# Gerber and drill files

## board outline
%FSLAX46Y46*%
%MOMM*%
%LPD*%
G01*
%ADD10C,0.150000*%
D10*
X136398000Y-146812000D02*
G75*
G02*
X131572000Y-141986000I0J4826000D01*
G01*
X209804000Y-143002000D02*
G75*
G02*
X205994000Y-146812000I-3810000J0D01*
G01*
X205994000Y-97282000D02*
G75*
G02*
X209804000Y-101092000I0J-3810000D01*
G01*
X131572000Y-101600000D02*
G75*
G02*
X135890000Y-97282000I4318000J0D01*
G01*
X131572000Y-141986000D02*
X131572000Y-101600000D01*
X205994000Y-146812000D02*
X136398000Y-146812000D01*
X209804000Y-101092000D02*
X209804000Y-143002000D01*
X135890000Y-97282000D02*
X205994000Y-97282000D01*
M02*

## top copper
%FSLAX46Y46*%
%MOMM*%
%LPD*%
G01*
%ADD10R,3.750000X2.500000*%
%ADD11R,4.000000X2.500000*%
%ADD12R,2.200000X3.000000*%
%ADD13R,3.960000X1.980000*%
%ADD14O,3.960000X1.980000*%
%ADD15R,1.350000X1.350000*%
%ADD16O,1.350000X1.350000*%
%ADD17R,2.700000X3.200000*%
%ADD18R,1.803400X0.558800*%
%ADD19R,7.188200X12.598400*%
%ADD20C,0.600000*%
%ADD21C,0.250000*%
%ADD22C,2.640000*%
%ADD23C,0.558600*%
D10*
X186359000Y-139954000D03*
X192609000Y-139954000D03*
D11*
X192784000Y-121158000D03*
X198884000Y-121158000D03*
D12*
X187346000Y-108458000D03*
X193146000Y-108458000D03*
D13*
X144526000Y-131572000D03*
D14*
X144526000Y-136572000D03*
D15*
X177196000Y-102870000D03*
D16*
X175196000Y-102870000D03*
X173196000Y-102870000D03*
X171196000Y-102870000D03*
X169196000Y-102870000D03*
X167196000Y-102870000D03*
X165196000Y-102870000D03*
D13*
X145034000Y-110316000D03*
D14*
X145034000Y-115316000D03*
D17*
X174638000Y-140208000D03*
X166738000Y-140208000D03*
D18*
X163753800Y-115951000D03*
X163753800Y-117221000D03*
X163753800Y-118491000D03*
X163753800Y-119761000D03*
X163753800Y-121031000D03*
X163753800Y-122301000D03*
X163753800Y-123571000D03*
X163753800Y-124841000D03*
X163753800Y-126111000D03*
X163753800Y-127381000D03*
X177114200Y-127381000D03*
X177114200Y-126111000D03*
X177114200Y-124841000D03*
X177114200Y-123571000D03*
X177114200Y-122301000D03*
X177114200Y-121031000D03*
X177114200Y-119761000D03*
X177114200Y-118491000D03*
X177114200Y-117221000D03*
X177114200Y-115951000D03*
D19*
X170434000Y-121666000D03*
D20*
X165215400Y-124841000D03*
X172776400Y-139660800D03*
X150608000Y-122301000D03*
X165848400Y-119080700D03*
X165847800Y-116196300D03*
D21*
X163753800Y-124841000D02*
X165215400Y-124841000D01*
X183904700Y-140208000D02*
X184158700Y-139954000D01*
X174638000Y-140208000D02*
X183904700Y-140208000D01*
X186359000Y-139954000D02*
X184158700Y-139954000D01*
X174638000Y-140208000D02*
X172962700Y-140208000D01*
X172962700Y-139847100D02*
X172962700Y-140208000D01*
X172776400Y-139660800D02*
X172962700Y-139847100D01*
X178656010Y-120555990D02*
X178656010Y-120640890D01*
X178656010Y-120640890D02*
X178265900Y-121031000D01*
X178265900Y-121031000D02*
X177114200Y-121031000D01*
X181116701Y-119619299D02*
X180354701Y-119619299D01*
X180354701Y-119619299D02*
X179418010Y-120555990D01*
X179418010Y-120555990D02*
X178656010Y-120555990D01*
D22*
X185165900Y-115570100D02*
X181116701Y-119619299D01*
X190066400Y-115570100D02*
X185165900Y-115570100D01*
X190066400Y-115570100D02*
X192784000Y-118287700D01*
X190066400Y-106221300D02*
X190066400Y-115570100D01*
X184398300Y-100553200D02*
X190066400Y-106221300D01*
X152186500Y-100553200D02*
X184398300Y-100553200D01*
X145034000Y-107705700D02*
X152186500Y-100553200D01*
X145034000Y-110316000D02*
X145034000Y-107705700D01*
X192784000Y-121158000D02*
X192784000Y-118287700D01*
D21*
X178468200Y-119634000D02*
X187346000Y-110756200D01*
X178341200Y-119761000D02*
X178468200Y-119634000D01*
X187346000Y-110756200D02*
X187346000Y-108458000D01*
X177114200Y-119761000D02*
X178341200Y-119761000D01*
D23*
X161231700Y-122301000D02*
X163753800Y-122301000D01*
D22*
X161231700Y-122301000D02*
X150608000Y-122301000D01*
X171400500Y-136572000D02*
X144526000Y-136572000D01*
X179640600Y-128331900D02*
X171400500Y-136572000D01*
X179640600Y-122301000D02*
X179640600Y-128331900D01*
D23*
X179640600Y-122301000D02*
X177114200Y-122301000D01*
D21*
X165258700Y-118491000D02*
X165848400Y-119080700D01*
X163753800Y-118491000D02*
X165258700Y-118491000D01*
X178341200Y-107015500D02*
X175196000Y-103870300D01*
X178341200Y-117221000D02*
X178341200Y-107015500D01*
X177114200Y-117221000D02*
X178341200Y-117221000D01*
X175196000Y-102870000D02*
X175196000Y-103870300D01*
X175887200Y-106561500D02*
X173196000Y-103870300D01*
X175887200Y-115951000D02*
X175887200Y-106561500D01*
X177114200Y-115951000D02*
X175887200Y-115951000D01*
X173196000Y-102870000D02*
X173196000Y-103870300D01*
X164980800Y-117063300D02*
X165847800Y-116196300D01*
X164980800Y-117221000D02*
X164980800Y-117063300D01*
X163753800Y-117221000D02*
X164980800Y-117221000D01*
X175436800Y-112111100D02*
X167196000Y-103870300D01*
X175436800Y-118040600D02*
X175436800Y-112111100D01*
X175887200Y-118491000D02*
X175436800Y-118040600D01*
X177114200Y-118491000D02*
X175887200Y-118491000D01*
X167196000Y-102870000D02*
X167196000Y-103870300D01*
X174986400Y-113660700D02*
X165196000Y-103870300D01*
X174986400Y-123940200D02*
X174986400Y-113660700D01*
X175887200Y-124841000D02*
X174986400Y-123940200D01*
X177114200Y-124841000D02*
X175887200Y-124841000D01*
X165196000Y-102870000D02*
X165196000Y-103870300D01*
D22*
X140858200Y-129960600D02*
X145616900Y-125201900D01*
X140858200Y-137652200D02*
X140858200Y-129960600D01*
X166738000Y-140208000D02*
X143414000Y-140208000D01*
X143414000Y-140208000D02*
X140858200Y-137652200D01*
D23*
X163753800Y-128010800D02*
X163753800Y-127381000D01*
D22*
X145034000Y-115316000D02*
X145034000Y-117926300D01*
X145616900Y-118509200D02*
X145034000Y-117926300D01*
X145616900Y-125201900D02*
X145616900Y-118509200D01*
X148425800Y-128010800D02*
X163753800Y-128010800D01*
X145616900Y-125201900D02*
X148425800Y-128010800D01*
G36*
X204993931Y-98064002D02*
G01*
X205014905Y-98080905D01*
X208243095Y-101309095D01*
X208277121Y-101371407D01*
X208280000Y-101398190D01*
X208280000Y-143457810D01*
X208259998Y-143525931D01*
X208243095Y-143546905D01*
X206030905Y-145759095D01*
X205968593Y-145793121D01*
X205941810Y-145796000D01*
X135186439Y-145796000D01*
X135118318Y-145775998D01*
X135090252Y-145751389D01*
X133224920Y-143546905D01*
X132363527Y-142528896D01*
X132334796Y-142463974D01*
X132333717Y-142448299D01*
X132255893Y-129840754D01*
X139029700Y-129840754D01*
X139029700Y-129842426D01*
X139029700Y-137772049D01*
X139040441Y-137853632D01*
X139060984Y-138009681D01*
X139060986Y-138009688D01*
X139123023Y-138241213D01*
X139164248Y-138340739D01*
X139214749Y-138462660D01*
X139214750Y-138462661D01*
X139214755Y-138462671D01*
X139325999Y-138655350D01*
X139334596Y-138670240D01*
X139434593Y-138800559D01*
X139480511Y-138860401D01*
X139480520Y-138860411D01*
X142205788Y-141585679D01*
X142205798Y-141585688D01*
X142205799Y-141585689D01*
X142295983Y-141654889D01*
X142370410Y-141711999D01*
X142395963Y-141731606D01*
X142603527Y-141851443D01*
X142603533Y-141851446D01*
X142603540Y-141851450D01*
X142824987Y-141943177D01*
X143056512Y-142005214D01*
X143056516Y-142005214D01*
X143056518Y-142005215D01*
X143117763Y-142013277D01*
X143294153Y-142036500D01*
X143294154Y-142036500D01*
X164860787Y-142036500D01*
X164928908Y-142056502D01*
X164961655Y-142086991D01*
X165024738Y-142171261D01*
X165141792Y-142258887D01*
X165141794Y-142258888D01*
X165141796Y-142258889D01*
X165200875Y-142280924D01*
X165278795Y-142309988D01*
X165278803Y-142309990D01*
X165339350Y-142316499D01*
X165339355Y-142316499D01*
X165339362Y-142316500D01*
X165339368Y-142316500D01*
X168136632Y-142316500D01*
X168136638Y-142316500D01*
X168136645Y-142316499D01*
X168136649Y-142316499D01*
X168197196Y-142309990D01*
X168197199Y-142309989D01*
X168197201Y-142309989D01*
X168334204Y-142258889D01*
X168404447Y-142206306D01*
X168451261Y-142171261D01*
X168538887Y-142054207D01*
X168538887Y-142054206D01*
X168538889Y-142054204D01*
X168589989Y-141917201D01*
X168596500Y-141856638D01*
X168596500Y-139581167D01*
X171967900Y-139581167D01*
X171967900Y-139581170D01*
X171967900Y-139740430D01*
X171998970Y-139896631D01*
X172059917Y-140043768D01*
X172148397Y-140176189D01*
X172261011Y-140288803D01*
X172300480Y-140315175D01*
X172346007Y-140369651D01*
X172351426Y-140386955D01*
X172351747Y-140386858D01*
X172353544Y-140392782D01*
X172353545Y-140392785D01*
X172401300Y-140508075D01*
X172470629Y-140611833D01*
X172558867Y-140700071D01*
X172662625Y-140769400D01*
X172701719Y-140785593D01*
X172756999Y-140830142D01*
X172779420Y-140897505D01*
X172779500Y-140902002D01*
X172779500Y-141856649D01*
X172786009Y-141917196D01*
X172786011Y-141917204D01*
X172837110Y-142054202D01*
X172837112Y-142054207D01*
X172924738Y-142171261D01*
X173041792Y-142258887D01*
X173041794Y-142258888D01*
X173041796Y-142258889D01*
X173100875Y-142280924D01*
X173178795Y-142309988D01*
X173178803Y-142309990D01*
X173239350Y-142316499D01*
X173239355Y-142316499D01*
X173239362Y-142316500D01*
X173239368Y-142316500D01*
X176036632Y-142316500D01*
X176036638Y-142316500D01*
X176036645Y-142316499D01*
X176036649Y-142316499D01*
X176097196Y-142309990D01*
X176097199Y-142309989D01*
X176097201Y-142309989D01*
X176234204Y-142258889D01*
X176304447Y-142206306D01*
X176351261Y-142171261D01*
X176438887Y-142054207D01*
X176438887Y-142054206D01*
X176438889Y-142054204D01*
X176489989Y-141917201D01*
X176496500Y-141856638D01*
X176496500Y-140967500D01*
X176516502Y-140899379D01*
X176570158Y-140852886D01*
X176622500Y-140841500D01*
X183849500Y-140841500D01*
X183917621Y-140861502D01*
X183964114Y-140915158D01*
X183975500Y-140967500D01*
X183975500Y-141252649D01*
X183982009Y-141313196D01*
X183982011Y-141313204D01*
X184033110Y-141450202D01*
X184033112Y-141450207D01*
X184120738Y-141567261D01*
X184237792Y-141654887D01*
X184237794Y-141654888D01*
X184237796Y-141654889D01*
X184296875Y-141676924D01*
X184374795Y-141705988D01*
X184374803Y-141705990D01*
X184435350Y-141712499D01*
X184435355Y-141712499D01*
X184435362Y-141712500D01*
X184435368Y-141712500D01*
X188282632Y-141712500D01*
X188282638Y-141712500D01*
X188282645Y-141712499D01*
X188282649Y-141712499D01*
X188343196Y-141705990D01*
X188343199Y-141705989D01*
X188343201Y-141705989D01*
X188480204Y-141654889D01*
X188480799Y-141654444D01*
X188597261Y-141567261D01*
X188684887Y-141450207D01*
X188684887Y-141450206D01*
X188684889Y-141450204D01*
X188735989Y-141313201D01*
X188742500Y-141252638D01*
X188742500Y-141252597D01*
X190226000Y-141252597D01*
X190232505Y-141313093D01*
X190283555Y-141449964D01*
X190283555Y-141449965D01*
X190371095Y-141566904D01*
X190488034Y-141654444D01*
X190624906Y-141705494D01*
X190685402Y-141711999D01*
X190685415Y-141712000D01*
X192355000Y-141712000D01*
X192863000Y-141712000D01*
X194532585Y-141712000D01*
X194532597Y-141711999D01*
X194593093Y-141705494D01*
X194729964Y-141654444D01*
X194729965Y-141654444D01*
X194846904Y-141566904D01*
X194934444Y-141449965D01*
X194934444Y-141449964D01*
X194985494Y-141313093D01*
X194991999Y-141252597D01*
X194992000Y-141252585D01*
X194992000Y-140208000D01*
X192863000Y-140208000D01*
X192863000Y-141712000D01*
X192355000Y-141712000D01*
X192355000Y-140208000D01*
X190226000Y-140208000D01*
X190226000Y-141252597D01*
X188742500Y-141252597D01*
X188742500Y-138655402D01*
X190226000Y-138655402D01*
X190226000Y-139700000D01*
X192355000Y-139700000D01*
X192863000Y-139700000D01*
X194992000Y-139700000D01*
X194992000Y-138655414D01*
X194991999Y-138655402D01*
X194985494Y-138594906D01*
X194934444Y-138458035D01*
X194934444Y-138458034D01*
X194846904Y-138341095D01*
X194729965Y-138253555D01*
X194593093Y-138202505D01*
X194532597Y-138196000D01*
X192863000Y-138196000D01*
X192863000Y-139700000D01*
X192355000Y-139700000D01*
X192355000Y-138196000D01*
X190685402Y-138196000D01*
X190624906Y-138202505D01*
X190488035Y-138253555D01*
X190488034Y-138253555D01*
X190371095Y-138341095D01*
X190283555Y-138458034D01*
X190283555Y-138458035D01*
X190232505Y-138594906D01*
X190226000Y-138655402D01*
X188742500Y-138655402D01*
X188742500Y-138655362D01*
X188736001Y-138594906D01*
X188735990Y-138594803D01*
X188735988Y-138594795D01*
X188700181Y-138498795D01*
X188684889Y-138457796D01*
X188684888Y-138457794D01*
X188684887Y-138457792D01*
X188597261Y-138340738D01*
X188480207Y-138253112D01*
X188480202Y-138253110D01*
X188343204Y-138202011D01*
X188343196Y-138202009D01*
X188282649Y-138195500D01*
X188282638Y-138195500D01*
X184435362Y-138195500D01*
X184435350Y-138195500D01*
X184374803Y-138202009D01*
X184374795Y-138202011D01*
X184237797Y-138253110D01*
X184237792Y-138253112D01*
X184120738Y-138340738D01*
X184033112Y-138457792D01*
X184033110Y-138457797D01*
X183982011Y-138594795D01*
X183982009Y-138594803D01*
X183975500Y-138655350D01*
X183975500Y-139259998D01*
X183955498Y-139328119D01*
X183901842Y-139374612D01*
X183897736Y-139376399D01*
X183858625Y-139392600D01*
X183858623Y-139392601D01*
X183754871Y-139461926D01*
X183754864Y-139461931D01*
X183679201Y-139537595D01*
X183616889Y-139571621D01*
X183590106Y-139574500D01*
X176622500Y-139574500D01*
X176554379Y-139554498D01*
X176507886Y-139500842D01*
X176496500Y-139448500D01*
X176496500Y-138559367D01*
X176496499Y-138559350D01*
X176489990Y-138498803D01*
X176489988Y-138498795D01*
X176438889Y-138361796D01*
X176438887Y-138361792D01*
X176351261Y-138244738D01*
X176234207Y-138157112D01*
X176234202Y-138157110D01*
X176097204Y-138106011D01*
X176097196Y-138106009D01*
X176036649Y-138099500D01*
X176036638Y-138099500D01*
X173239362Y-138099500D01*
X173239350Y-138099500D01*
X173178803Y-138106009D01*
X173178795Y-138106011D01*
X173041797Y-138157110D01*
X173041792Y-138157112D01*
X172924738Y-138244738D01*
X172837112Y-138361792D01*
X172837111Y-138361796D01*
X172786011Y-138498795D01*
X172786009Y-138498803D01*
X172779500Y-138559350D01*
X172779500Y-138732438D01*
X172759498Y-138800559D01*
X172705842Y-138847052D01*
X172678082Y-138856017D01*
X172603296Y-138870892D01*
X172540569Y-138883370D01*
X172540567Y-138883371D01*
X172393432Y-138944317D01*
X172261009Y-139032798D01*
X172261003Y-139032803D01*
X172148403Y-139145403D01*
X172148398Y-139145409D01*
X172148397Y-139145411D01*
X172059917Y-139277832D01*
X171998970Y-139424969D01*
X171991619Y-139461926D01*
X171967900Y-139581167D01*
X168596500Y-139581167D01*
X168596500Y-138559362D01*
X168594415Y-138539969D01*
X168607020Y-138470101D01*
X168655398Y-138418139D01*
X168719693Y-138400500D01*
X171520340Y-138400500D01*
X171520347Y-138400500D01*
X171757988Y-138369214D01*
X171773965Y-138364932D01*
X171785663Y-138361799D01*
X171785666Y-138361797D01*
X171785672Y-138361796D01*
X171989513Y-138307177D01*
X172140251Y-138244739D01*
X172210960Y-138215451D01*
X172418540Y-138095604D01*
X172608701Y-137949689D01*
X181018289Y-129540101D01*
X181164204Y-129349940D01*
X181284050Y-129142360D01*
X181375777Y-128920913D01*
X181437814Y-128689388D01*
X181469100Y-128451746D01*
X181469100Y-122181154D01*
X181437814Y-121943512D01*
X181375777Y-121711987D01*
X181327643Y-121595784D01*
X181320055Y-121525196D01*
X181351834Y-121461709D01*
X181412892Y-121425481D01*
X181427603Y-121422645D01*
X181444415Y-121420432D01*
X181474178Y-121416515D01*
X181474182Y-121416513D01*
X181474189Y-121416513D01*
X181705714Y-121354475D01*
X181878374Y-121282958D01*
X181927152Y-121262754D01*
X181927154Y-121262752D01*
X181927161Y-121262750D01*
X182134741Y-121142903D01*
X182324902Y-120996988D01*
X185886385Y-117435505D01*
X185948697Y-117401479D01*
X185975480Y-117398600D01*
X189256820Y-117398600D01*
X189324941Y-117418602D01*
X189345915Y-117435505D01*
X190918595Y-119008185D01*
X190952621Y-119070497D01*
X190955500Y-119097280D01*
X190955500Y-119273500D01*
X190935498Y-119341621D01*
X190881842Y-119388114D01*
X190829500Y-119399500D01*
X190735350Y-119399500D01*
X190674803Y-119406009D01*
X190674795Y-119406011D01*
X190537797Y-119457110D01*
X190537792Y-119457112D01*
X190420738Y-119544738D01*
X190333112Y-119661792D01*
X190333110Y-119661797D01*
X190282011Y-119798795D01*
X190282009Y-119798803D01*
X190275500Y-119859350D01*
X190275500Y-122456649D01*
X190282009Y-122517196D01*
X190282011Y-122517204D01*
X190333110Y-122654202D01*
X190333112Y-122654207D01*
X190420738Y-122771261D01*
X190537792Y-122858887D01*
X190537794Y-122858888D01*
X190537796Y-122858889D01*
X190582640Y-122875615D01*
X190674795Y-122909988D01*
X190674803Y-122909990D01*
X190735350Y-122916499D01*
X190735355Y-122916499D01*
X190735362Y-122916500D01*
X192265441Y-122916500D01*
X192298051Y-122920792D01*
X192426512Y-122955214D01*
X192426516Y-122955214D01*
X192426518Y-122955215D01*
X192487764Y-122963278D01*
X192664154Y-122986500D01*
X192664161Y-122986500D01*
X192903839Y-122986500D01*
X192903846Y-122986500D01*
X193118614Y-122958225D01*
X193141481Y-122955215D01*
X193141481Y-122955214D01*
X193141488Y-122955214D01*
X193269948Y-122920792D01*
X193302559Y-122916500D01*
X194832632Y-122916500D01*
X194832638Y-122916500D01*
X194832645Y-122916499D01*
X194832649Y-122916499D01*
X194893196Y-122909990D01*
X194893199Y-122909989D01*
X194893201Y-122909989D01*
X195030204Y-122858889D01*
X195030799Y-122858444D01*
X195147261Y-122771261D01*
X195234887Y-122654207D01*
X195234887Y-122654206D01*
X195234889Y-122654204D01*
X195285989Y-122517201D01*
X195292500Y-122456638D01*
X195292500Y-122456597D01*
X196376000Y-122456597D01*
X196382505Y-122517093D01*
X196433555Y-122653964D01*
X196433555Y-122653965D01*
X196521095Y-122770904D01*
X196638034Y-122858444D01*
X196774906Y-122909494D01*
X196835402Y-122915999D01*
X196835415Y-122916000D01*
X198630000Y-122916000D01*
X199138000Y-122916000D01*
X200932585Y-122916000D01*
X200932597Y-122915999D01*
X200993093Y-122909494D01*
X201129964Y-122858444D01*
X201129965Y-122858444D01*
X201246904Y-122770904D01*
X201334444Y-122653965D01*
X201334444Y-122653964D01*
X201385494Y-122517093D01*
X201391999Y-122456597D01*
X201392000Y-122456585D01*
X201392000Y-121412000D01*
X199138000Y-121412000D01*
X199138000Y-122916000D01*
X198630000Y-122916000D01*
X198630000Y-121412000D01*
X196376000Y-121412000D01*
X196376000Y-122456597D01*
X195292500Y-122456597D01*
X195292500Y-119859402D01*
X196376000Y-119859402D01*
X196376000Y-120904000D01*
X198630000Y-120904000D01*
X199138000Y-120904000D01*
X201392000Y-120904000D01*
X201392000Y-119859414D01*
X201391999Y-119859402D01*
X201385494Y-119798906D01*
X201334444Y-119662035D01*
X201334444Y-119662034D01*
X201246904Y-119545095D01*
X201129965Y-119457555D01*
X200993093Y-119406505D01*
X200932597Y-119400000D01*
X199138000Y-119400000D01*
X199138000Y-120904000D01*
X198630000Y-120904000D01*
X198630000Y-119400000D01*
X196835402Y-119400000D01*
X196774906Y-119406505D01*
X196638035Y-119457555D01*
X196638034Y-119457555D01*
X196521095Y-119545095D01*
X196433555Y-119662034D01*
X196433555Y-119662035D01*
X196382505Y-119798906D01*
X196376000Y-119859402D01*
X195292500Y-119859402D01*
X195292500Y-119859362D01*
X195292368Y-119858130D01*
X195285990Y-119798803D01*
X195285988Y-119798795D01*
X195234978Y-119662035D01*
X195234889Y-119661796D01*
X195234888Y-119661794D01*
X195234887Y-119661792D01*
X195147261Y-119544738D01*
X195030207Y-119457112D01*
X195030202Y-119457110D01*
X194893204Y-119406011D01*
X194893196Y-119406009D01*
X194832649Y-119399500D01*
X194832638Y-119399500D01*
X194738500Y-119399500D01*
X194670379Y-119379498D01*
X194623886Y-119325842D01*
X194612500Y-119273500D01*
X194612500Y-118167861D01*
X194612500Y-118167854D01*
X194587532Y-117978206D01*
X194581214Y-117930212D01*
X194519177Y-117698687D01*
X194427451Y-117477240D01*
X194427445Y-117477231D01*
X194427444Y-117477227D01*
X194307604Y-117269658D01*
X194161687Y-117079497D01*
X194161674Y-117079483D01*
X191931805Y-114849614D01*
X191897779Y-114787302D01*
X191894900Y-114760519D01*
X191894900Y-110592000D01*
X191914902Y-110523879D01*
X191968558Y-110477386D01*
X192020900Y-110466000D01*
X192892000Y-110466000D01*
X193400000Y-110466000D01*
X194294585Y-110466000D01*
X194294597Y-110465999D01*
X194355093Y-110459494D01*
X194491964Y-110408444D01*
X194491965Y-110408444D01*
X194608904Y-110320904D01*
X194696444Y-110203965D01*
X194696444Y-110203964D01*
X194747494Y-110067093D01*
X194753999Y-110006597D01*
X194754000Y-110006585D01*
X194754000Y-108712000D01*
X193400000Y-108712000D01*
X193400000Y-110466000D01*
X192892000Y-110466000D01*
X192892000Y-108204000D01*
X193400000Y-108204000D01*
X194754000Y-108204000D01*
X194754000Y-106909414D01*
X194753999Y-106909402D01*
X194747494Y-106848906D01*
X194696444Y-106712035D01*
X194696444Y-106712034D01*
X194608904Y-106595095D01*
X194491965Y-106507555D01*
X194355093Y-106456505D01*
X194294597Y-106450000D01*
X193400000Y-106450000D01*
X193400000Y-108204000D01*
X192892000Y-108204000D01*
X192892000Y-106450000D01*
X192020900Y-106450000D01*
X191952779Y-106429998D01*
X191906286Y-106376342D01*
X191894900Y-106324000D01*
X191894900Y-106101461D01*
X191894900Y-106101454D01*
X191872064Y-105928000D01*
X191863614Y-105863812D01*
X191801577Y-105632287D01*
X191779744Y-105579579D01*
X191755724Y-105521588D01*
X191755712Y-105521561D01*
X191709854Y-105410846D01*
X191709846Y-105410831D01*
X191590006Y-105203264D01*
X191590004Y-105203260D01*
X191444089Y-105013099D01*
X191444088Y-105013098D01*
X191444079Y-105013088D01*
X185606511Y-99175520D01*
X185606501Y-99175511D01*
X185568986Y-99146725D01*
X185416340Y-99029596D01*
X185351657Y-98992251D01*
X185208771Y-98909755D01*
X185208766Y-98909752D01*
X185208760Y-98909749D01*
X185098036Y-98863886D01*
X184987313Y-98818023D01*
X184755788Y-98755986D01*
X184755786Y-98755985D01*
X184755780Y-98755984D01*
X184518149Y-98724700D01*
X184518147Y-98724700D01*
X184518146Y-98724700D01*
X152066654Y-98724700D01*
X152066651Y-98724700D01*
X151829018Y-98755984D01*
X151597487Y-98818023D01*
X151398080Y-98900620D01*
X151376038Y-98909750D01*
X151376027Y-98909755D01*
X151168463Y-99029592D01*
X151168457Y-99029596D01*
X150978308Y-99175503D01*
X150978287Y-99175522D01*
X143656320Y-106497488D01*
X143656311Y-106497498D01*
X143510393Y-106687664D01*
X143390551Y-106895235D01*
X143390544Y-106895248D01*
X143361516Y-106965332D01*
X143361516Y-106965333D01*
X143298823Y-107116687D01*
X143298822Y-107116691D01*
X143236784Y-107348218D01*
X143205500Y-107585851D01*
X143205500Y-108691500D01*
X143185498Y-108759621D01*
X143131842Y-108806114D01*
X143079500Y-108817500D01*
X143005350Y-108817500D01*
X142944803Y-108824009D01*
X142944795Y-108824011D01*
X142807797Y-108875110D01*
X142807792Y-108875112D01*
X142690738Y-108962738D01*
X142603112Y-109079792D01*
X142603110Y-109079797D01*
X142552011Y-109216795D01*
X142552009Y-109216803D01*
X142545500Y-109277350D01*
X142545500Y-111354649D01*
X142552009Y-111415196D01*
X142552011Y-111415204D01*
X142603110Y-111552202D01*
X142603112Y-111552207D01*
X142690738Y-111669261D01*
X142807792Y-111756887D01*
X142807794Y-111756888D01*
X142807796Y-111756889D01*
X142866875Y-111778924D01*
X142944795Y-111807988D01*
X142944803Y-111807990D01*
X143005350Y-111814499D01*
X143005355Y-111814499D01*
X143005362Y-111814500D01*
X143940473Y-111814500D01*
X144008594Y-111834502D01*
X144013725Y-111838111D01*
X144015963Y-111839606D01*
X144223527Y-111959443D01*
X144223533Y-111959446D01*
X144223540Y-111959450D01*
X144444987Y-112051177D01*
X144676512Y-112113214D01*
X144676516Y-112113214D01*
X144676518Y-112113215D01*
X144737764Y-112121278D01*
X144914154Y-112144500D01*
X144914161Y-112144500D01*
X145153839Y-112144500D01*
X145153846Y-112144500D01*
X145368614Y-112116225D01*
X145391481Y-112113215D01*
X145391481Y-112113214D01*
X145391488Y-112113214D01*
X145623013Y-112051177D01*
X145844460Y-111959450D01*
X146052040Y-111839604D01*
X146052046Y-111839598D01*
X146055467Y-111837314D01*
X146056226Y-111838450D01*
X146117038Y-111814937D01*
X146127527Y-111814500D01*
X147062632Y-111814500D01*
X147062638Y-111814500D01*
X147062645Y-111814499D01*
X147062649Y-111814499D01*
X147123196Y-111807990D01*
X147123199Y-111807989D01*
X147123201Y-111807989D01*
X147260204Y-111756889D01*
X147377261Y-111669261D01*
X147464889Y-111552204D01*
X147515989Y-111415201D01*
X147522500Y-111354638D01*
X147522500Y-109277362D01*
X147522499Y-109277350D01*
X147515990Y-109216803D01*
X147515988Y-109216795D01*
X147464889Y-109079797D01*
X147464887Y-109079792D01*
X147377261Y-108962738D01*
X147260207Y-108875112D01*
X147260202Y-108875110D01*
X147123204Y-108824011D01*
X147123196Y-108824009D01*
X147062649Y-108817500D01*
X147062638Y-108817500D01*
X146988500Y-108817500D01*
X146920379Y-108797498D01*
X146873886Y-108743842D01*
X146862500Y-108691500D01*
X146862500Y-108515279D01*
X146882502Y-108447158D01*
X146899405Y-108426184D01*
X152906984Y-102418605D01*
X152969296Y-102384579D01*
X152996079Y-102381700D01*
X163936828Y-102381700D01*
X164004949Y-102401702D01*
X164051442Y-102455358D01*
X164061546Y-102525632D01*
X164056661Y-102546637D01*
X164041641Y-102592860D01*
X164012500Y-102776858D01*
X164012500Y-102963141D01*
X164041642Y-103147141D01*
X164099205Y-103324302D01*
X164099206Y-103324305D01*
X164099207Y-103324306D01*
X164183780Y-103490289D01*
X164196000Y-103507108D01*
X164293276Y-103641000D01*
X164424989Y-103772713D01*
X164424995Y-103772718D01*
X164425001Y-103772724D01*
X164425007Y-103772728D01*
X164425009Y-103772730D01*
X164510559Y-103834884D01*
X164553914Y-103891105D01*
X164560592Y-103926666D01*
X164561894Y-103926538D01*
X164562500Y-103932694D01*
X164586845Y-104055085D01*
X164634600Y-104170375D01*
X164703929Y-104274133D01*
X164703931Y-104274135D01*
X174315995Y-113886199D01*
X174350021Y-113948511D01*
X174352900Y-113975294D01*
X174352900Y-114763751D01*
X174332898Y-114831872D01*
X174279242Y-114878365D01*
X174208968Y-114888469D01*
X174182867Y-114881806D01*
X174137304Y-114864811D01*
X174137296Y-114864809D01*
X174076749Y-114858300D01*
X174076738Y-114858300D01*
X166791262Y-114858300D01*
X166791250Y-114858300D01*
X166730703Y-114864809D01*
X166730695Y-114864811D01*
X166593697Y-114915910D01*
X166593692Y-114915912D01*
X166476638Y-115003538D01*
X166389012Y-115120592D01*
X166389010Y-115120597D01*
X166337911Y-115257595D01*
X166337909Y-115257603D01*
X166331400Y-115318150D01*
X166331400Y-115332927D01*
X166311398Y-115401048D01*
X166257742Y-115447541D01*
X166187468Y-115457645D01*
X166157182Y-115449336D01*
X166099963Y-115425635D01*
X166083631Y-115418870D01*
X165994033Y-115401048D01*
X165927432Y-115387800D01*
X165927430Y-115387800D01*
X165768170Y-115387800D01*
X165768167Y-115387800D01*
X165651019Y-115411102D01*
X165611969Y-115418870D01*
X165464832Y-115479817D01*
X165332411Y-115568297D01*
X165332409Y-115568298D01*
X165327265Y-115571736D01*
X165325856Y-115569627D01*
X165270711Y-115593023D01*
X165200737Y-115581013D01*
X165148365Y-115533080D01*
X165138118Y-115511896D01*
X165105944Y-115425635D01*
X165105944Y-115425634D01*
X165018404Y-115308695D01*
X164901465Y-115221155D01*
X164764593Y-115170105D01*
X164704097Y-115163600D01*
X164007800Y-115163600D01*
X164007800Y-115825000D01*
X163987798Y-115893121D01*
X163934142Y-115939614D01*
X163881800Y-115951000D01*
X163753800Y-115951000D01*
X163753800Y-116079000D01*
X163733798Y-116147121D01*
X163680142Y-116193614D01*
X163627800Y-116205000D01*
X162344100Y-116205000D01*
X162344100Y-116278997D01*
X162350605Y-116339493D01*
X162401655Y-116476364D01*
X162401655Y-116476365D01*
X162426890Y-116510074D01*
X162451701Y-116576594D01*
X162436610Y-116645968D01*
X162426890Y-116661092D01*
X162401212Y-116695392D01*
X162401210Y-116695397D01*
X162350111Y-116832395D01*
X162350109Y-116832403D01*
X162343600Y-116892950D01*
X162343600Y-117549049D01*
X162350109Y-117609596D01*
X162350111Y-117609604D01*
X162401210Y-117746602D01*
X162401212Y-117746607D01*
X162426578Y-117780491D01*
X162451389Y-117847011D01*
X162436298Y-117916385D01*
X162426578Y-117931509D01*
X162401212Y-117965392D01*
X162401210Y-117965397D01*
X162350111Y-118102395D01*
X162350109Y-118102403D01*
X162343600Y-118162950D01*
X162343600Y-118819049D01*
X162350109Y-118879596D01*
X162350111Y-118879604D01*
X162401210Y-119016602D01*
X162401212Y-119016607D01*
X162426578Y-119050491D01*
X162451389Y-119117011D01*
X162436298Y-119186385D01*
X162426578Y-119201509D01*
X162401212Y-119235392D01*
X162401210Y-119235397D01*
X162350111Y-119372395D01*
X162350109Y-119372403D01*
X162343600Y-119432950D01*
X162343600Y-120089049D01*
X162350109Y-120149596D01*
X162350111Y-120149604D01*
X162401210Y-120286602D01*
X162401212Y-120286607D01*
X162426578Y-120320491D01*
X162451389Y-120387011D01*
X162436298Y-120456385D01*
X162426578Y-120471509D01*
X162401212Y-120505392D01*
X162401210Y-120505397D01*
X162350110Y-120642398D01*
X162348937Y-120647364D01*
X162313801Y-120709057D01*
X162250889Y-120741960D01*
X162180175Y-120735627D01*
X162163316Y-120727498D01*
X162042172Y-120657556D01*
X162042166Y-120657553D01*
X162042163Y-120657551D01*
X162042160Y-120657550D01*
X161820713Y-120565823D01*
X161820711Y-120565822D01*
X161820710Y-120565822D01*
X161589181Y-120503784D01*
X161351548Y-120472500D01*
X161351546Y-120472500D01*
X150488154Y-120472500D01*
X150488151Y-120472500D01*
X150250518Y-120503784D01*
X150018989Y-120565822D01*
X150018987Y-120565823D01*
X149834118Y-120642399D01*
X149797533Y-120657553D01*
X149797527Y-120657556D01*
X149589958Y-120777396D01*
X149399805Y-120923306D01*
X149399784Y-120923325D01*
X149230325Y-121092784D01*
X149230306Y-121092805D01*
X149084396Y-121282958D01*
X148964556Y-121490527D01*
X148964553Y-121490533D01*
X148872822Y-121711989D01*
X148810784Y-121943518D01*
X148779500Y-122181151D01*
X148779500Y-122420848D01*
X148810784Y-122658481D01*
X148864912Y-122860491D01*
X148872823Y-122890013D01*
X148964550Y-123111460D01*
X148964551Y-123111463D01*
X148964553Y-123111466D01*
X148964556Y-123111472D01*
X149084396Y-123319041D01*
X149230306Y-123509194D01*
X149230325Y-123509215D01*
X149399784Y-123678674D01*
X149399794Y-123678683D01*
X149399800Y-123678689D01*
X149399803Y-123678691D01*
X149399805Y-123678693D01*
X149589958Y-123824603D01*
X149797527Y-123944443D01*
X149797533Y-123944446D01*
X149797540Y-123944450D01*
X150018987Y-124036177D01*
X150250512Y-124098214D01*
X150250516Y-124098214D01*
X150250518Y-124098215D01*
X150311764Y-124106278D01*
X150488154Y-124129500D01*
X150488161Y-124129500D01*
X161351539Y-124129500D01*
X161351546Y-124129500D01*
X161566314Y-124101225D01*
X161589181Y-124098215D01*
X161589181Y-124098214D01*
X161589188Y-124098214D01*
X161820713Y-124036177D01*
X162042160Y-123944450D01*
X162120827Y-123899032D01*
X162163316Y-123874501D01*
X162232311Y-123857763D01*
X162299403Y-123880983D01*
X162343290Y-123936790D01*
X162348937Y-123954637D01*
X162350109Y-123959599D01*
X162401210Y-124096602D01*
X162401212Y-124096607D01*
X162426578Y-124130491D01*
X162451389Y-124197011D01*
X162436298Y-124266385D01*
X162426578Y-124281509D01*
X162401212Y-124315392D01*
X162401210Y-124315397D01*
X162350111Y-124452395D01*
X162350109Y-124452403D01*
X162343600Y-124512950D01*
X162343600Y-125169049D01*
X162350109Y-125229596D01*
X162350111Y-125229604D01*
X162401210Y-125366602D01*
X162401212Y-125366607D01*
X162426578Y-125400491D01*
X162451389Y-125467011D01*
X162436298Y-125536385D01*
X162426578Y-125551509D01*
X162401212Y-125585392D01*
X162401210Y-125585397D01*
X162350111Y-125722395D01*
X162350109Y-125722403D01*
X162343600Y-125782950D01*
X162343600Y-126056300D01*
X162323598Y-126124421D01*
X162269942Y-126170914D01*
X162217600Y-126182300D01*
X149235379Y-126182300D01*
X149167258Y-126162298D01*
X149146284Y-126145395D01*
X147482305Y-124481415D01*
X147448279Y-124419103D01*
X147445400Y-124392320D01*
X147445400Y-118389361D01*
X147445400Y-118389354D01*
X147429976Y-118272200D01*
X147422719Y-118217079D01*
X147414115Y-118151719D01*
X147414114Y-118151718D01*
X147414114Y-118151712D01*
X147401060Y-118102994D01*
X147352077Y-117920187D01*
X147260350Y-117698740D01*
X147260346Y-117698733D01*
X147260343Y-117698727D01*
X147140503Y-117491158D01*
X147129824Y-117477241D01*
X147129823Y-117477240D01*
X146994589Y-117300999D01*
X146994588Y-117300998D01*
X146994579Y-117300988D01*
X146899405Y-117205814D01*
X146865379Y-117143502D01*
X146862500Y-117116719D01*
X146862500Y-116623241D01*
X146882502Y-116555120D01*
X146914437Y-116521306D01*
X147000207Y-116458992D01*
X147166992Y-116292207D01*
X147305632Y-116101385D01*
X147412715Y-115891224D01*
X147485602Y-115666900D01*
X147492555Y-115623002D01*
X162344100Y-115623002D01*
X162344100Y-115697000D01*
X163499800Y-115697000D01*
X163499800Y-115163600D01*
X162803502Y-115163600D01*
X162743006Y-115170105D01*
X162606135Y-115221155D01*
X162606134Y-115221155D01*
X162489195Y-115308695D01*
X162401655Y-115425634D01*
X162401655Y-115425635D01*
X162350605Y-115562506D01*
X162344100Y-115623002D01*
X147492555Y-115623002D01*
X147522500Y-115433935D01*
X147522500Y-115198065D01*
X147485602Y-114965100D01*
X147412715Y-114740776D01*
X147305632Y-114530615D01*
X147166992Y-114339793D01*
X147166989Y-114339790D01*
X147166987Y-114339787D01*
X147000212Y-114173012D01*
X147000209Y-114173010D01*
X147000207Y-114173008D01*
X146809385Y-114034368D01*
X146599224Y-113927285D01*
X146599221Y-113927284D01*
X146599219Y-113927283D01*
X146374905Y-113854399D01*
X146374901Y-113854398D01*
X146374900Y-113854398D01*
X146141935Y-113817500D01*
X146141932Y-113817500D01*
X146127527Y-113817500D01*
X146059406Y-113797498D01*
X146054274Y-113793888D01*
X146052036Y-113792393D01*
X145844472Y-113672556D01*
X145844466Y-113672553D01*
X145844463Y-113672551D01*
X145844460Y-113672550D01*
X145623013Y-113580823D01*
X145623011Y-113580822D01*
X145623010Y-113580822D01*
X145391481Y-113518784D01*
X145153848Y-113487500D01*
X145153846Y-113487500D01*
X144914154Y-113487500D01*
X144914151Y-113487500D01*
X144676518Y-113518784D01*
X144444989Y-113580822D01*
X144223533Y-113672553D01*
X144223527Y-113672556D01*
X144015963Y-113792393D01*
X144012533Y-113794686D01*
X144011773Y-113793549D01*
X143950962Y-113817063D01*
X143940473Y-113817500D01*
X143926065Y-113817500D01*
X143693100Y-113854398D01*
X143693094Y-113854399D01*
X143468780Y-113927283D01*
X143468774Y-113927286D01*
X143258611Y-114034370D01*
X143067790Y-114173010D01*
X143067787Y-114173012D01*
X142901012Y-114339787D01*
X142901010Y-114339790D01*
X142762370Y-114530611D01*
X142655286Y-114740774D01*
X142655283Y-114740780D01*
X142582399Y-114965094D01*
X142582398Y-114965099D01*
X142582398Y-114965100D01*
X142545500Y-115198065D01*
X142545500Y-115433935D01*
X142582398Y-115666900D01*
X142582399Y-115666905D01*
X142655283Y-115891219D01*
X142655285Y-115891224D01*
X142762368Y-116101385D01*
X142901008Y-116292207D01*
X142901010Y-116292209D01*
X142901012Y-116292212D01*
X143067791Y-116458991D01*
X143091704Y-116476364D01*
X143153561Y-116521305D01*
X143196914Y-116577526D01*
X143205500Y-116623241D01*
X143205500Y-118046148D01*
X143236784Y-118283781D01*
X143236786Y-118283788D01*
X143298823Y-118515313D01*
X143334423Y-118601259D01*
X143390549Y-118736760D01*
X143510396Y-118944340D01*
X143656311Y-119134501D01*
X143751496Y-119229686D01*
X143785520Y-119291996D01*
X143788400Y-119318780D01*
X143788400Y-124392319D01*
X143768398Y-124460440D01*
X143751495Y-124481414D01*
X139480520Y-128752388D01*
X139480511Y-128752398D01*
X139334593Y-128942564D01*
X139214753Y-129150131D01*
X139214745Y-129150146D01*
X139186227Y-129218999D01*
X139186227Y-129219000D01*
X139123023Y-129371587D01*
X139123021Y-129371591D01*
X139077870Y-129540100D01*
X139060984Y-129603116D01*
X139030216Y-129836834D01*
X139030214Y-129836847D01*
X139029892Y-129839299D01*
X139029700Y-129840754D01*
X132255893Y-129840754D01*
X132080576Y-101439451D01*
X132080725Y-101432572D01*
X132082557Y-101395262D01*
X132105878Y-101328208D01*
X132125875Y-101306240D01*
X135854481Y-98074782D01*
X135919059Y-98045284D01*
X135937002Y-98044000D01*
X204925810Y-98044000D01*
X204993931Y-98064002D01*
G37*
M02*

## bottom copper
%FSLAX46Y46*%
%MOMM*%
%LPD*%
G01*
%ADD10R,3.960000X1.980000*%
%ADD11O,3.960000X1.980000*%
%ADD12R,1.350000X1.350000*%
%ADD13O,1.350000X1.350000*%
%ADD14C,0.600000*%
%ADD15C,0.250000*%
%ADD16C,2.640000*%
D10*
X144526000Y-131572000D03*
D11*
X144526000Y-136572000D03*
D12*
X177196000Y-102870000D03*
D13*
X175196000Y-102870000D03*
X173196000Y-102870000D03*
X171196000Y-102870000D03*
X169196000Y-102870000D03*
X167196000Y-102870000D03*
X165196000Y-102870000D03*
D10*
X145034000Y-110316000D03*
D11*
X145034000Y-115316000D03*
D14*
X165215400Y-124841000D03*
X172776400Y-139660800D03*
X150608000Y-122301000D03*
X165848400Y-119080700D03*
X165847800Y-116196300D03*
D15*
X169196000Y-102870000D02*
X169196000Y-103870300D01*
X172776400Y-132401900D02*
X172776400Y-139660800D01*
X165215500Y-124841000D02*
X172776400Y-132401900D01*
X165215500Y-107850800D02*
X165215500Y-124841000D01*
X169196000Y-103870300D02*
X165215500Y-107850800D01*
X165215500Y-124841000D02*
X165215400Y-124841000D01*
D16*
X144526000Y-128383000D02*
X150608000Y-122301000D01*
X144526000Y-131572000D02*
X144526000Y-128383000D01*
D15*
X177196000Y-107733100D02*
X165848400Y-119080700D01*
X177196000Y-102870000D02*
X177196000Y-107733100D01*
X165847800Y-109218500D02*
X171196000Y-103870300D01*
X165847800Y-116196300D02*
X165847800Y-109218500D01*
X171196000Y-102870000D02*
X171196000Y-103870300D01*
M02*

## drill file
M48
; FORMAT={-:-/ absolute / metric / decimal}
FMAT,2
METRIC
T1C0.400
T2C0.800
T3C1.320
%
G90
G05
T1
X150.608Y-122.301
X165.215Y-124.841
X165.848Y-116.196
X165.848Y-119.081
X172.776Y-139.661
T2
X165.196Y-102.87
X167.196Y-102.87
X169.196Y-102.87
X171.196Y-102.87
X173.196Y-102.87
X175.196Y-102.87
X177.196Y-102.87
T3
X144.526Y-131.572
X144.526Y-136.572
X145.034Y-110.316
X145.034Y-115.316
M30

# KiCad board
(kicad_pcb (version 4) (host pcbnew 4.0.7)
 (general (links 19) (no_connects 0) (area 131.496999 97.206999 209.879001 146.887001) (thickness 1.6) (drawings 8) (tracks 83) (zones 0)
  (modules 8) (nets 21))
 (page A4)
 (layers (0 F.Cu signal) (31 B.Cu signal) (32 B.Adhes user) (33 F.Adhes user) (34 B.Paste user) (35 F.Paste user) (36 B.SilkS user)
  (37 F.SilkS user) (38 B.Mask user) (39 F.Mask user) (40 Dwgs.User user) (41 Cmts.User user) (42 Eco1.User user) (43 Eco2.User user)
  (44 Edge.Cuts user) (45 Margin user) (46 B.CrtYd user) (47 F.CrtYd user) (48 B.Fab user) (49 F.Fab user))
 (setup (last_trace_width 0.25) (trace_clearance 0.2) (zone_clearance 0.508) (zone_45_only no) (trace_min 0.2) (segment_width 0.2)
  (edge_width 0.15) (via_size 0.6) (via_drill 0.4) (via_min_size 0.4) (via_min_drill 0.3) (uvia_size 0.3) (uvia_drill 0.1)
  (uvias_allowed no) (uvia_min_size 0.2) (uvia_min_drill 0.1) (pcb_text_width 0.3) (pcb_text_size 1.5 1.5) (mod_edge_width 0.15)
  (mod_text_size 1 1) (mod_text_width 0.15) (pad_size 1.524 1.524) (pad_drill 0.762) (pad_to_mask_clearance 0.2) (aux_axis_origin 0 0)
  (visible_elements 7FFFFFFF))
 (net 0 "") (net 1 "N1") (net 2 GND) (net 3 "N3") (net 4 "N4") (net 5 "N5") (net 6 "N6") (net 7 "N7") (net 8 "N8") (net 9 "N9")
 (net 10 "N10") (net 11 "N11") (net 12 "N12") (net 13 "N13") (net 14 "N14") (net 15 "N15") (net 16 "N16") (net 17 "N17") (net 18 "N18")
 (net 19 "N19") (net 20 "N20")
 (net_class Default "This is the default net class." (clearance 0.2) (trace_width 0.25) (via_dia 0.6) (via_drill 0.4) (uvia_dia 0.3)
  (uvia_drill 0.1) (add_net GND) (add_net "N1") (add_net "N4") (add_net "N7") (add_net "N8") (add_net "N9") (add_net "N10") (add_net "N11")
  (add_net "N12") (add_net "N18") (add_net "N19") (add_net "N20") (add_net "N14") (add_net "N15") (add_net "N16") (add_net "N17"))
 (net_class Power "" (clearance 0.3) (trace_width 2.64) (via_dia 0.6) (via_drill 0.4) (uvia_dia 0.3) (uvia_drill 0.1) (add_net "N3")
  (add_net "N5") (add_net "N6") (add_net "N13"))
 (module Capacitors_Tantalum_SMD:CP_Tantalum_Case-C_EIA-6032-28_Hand (layer F.Cu) (at 189.484 139.954)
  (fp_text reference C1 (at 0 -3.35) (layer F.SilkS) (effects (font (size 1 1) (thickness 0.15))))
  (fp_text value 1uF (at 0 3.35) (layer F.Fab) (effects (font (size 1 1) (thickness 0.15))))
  (pad 1 smd rect (at -3.125 0) (size 3.75 2.5) (layers F.Cu F.Paste F.Mask) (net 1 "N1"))
  (pad 2 smd rect (at 3.125 0) (size 3.75 2.5) (layers F.Cu F.Paste F.Mask) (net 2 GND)))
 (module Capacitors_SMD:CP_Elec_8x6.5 (layer F.Cu) (at 195.834 121.158)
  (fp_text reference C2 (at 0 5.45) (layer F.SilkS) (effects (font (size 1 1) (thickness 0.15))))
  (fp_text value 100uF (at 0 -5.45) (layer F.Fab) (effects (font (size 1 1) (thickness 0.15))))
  (pad 1 smd rect (at -3.05 0 180) (size 4 2.5) (layers F.Cu F.Paste F.Mask) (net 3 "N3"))
  (pad 2 smd rect (at 3.05 0 180) (size 4 2.5) (layers F.Cu F.Paste F.Mask) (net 2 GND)))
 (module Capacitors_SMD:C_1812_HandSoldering (layer F.Cu) (at 190.246 108.458)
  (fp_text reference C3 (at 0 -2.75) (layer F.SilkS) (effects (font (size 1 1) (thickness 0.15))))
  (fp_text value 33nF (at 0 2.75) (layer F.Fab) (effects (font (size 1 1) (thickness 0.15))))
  (pad 1 smd rect (at -2.9 0) (size 2.2 3) (layers F.Cu F.Paste F.Mask) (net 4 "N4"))
  (pad 2 smd rect (at 2.9 0) (size 2.2 3) (layers F.Cu F.Paste F.Mask) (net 2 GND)))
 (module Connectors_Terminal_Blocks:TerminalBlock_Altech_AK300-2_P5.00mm (layer F.Cu) (at 144.526 131.572 270)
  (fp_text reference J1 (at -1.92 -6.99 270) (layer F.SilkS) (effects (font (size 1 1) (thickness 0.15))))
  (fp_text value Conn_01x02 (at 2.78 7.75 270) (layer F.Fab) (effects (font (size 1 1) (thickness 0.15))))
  (pad 1 thru_hole rect (at 0 0 270) (size 1.98 3.96) (drill 1.32) (layers *.Cu *.Mask) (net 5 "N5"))
  (pad 2 thru_hole oval (at 5 0 270) (size 1.98 3.96) (drill 1.32) (layers *.Cu *.Mask) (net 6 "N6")))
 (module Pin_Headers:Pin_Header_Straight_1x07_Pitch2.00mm (layer F.Cu) (at 177.196 102.87 270)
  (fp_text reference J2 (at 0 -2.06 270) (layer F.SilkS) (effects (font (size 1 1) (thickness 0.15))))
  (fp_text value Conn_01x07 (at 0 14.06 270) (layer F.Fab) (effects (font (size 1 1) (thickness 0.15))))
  (pad 1 thru_hole rect (at 0 0 270) (size 1.35 1.35) (drill 0.8) (layers *.Cu *.Mask) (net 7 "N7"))
  (pad 2 thru_hole oval (at 0 2 270) (size 1.35 1.35) (drill 0.8) (layers *.Cu *.Mask) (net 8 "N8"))
  (pad 3 thru_hole oval (at 0 4 270) (size 1.35 1.35) (drill 0.8) (layers *.Cu *.Mask) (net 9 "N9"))
  (pad 4 thru_hole oval (at 0 6 270) (size 1.35 1.35) (drill 0.8) (layers *.Cu *.Mask) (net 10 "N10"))
  (pad 5 thru_hole oval (at 0 8 270) (size 1.35 1.35) (drill 0.8) (layers *.Cu *.Mask) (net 1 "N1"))
  (pad 6 thru_hole oval (at 0 10 270) (size 1.35 1.35) (drill 0.8) (layers *.Cu *.Mask) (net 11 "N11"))
  (pad 7 thru_hole oval (at 0 12 270) (size 1.35 1.35) (drill 0.8) (layers *.Cu *.Mask) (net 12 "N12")))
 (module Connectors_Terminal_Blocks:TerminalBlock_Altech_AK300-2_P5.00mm (layer F.Cu) (at 145.034 110.316 270)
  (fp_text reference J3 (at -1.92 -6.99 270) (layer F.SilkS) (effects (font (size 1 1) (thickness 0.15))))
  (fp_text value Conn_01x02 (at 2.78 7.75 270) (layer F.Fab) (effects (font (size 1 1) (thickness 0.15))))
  (pad 1 thru_hole rect (at 0 0 270) (size 1.98 3.96) (drill 1.32) (layers *.Cu *.Mask) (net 3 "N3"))
  (pad 2 thru_hole oval (at 5 0 270) (size 1.98 3.96) (drill 1.32) (layers *.Cu *.Mask) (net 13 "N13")))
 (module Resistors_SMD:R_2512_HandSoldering (layer F.Cu) (at 170.688 140.208 180)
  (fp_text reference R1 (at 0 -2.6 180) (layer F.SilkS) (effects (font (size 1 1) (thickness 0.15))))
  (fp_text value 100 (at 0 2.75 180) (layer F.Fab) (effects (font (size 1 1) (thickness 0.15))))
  (pad 1 smd rect (at -3.95 0 180) (size 2.7 3.2) (layers F.Cu F.Paste F.Mask) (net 1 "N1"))
  (pad 2 smd rect (at 3.95 0 180) (size 2.7 3.2) (layers F.Cu F.Paste F.Mask) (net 13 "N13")))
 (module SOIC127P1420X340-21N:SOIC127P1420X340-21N (layer F.Cu) (at 170.434 121.666)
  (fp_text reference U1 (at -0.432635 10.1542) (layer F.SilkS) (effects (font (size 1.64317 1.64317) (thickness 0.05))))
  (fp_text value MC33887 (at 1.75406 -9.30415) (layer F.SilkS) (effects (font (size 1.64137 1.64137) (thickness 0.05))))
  (pad 1 smd rect (at -6.6802 -5.715) (size 1.8034 0.5588) (layers F.Cu F.Paste F.Mask) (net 2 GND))
  (pad 2 smd rect (at -6.6802 -4.445) (size 1.8034 0.5588) (layers F.Cu F.Paste F.Mask) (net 10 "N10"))
  (pad 3 smd rect (at -6.6802 -3.175) (size 1.8034 0.5588) (layers F.Cu F.Paste F.Mask) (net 7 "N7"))
  (pad 4 smd rect (at -6.6802 -1.905) (size 1.8034 0.5588) (layers F.Cu F.Paste F.Mask) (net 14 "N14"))
  (pad 5 smd rect (at -6.6802 -0.635) (size 1.8034 0.5588) (layers F.Cu F.Paste F.Mask) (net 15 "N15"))
  (pad 6 smd rect (at -6.6802 0.635) (size 1.8034 0.5588) (layers F.Cu F.Paste F.Mask) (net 5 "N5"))
  (pad 7 smd rect (at -6.6802 1.905) (size 1.8034 0.5588) (layers F.Cu F.Paste F.Mask) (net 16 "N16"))
  (pad 8 smd rect (at -6.6802 3.175) (size 1.8034 0.5588) (layers F.Cu F.Paste F.Mask) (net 1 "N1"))
  (pad 9 smd rect (at -6.6802 4.445) (size 1.8034 0.5588) (layers F.Cu F.Paste F.Mask) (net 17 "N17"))
  (pad 10 smd rect (at -6.6802 5.715) (size 1.8034 0.5588) (layers F.Cu F.Paste F.Mask) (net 13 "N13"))
  (pad 11 smd rect (at 6.6802 5.715) (size 1.8034 0.5588) (layers F.Cu F.Paste F.Mask) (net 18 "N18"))
  (pad 12 smd rect (at 6.6802 4.445) (size 1.8034 0.5588) (layers F.Cu F.Paste F.Mask) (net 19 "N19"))
  (pad 13 smd rect (at 6.6802 3.175) (size 1.8034 0.5588) (layers F.Cu F.Paste F.Mask) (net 12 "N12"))
  (pad 14 smd rect (at 6.6802 1.905) (size 1.8034 0.5588) (layers F.Cu F.Paste F.Mask) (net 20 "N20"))
  (pad 15 smd rect (at 6.6802 0.635) (size 1.8034 0.5588) (layers F.Cu F.Paste F.Mask) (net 6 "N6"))
  (pad 16 smd rect (at 6.6802 -0.635) (size 1.8034 0.5588) (layers F.Cu F.Paste F.Mask) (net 3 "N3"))
  (pad 17 smd rect (at 6.6802 -1.905) (size 1.8034 0.5588) (layers F.Cu F.Paste F.Mask) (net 4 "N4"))
  (pad 18 smd rect (at 6.6802 -3.175) (size 1.8034 0.5588) (layers F.Cu F.Paste F.Mask) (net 11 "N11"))
  (pad 19 smd rect (at 6.6802 -4.445) (size 1.8034 0.5588) (layers F.Cu F.Paste F.Mask) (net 8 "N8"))
  (pad 20 smd rect (at 6.6802 -5.715) (size 1.8034 0.5588) (layers F.Cu F.Paste F.Mask) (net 9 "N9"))
  (pad 21 smd rect (at 0 0) (size 7.1882 12.5984) (layers F.Cu F.Paste F.Mask)))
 (gr_arc (start 136.398 141.986) (end 136.398 146.812) (angle 90) (layer Edge.Cuts) (width 0.15))
 (gr_arc (start 205.994 143.002) (end 209.804 143.002) (angle 90) (layer Edge.Cuts) (width 0.15))
 (gr_arc (start 205.994 101.092) (end 205.994 97.282) (angle 90) (layer Edge.Cuts) (width 0.15))
 (gr_arc (start 135.89 101.6) (end 131.572 101.6) (angle 90) (layer Edge.Cuts) (width 0.15))
 (gr_line (start 131.572 141.986) (end 131.572 101.6) (layer Edge.Cuts) (width 0.15))
 (gr_line (start 205.994 146.812) (end 136.398 146.812) (layer Edge.Cuts) (width 0.15))
 (gr_line (start 209.804 101.092) (end 209.804 143.002) (layer Edge.Cuts) (width 0.15))
 (gr_line (start 135.89 97.282) (end 205.994 97.282) (layer Edge.Cuts) (width 0.15))
 (via (at 165.2154 124.841) (size 0.6) (layers F.Cu B.Cu) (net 1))
 (via (at 172.7764 139.6608) (size 0.6) (layers F.Cu B.Cu) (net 1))
 (segment (start 169.196 102.87) (end 169.196 103.8703) (width 0.25) (layer B.Cu) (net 1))
 (segment (start 163.7538 124.841) (end 165.2154 124.841) (width 0.25) (layer F.Cu) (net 1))
 (segment (start 183.9047 140.208) (end 184.1587 139.954) (width 0.25) (layer F.Cu) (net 1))
 (segment (start 174.638 140.208) (end 183.9047 140.208) (width 0.25) (layer F.Cu) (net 1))
 (segment (start 186.359 139.954) (end 184.1587 139.954) (width 0.25) (layer F.Cu) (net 1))
 (segment (start 174.638 140.208) (end 172.9627 140.208) (width 0.25) (layer F.Cu) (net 1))
 (segment (start 172.9627 139.8471) (end 172.9627 140.208) (width 0.25) (layer F.Cu) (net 1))
 (segment (start 172.7764 139.6608) (end 172.9627 139.8471) (width 0.25) (layer F.Cu) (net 1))
 (segment (start 172.7764 132.4019) (end 172.7764 139.6608) (width 0.25) (layer B.Cu) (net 1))
 (segment (start 165.2155 124.841) (end 172.7764 132.4019) (width 0.25) (layer B.Cu) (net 1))
 (segment (start 165.2155 107.8508) (end 165.2155 124.841) (width 0.25) (layer B.Cu) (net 1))
 (segment (start 169.196 103.8703) (end 165.2155 107.8508) (width 0.25) (layer B.Cu) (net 1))
 (segment (start 165.2155 124.841) (end 165.2154 124.841) (width 0.25) (layer B.Cu) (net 1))
 (segment (start 178.65601 120.55599) (end 178.65601 120.64089) (width 0.25) (layer F.Cu) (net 3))
 (segment (start 178.65601 120.64089) (end 178.2659 121.031) (width 0.25) (layer F.Cu) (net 3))
 (segment (start 178.2659 121.031) (end 177.1142 121.031) (width 0.25) (layer F.Cu) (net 3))
 (segment (start 181.116701 119.619299) (end 180.354701 119.619299) (width 0.25) (layer F.Cu) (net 3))
 (segment (start 180.354701 119.619299) (end 179.41801 120.55599) (width 0.25) (layer F.Cu) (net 3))
 (segment (start 179.41801 120.55599) (end 178.65601 120.55599) (width 0.25) (layer F.Cu) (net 3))
 (segment (start 185.1659 115.5701) (end 181.116701 119.619299) (width 2.64) (layer F.Cu) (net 3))
 (segment (start 190.0664 115.5701) (end 185.1659 115.5701) (width 2.64) (layer F.Cu) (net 3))
 (segment (start 190.0664 115.5701) (end 192.784 118.2877) (width 2.64) (layer F.Cu) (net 3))
 (segment (start 190.0664 106.2213) (end 190.0664 115.5701) (width 2.64) (layer F.Cu) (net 3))
 (segment (start 184.3983 100.5532) (end 190.0664 106.2213) (width 2.64) (layer F.Cu) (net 3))
 (segment (start 152.1865 100.5532) (end 184.3983 100.5532) (width 2.64) (layer F.Cu) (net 3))
 (segment (start 145.034 107.7057) (end 152.1865 100.5532) (width 2.64) (layer F.Cu) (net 3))
 (segment (start 145.034 110.316) (end 145.034 107.7057) (width 2.64) (layer F.Cu) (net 3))
 (segment (start 192.784 121.158) (end 192.784 118.2877) (width 2.64) (layer F.Cu) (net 3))
 (segment (start 178.4682 119.634) (end 187.346 110.7562) (width 0.25) (layer F.Cu) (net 4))
 (segment (start 178.3412 119.761) (end 178.4682 119.634) (width 0.25) (layer F.Cu) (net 4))
 (segment (start 187.346 110.7562) (end 187.346 108.458) (width 0.25) (layer F.Cu) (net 4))
 (segment (start 177.1142 119.761) (end 178.3412 119.761) (width 0.25) (layer F.Cu) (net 4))
 (via (at 150.608 122.301) (size 0.6) (layers F.Cu B.Cu) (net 5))
 (segment (start 161.2317 122.301) (end 163.7538 122.301) (width 0.5586) (layer F.Cu) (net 5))
 (segment (start 144.526 128.383) (end 150.608 122.301) (width 2.64) (layer B.Cu) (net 5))
 (segment (start 144.526 131.572) (end 144.526 128.383) (width 2.64) (layer B.Cu) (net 5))
 (segment (start 161.2317 122.301) (end 150.608 122.301) (width 2.64) (layer F.Cu) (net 5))
 (segment (start 171.4005 136.572) (end 144.526 136.572) (width 2.64) (layer F.Cu) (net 6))
 (segment (start 179.6406 128.3319) (end 171.4005 136.572) (width 2.64) (layer F.Cu) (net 6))
 (segment (start 179.6406 122.301) (end 179.6406 128.3319) (width 2.64) (layer F.Cu) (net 6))
 (segment (start 179.6406 122.301) (end 177.1142 122.301) (width 0.5586) (layer F.Cu) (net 6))
 (via (at 165.8484 119.0807) (size 0.6) (layers F.Cu B.Cu) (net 7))
 (segment (start 177.196 107.7331) (end 165.8484 119.0807) (width 0.25) (layer B.Cu) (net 7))
 (segment (start 177.196 102.87) (end 177.196 107.7331) (width 0.25) (layer B.Cu) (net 7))
 (segment (start 165.2587 118.491) (end 165.8484 119.0807) (width 0.25) (layer F.Cu) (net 7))
 (segment (start 163.7538 118.491) (end 165.2587 118.491) (width 0.25) (layer F.Cu) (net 7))
 (segment (start 178.3412 107.0155) (end 175.196 103.8703) (width 0.25) (layer F.Cu) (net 8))
 (segment (start 178.3412 117.221) (end 178.3412 107.0155) (width 0.25) (layer F.Cu) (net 8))
 (segment (start 177.1142 117.221) (end 178.3412 117.221) (width 0.25) (layer F.Cu) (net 8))
 (segment (start 175.196 102.87) (end 175.196 103.8703) (width 0.25) (layer F.Cu) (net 8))
 (segment (start 175.8872 106.5615) (end 173.196 103.8703) (width 0.25) (layer F.Cu) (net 9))
 (segment (start 175.8872 115.951) (end 175.8872 106.5615) (width 0.25) (layer F.Cu) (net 9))
 (segment (start 177.1142 115.951) (end 175.8872 115.951) (width 0.25) (layer F.Cu) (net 9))
 (segment (start 173.196 102.87) (end 173.196 103.8703) (width 0.25) (layer F.Cu) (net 9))
 (via (at 165.8478 116.1963) (size 0.6) (layers F.Cu B.Cu) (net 10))
 (segment (start 164.9808 117.0633) (end 165.8478 116.1963) (width 0.25) (layer F.Cu) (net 10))
 (segment (start 164.9808 117.221) (end 164.9808 117.0633) (width 0.25) (layer F.Cu) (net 10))
 (segment (start 165.8478 109.2185) (end 171.196 103.8703) (width 0.25) (layer B.Cu) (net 10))
 (segment (start 165.8478 116.1963) (end 165.8478 109.2185) (width 0.25) (layer B.Cu) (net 10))
 (segment (start 163.7538 117.221) (end 164.9808 117.221) (width 0.25) (layer F.Cu) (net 10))
 (segment (start 171.196 102.87) (end 171.196 103.8703) (width 0.25) (layer B.Cu) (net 10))
 (segment (start 175.4368 112.1111) (end 167.196 103.8703) (width 0.25) (layer F.Cu) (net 11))
 (segment (start 175.4368 118.0406) (end 175.4368 112.1111) (width 0.25) (layer F.Cu) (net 11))
 (segment (start 175.8872 118.491) (end 175.4368 118.0406) (width 0.25) (layer F.Cu) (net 11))
 (segment (start 177.1142 118.491) (end 175.8872 118.491) (width 0.25) (layer F.Cu) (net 11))
 (segment (start 167.196 102.87) (end 167.196 103.8703) (width 0.25) (layer F.Cu) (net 11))
 (segment (start 174.9864 113.6607) (end 165.196 103.8703) (width 0.25) (layer F.Cu) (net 12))
 (segment (start 174.9864 123.9402) (end 174.9864 113.6607) (width 0.25) (layer F.Cu) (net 12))
 (segment (start 175.8872 124.841) (end 174.9864 123.9402) (width 0.25) (layer F.Cu) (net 12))
 (segment (start 177.1142 124.841) (end 175.8872 124.841) (width 0.25) (layer F.Cu) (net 12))
 (segment (start 165.196 102.87) (end 165.196 103.8703) (width 0.25) (layer F.Cu) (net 12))
 (segment (start 140.8582 129.9606) (end 145.6169 125.2019) (width 2.64) (layer F.Cu) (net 13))
 (segment (start 140.8582 137.6522) (end 140.8582 129.9606) (width 2.64) (layer F.Cu) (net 13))
 (segment (start 166.738 140.208) (end 143.414 140.208) (width 2.64) (layer F.Cu) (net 13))
 (segment (start 143.414 140.208) (end 140.8582 137.6522) (width 2.64) (layer F.Cu) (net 13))
 (segment (start 163.7538 128.0108) (end 163.7538 127.381) (width 0.5586) (layer F.Cu) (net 13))
 (segment (start 145.034 115.316) (end 145.034 117.9263) (width 2.64) (layer F.Cu) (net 13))
 (segment (start 145.6169 118.5092) (end 145.034 117.9263) (width 2.64) (layer F.Cu) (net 13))
 (segment (start 145.6169 125.2019) (end 145.6169 118.5092) (width 2.64) (layer F.Cu) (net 13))
 (segment (start 148.4258 128.0108) (end 163.7538 128.0108) (width 2.64) (layer F.Cu) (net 13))
 (segment (start 145.6169 125.2019) (end 148.4258 128.0108) (width 2.64) (layer F.Cu) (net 13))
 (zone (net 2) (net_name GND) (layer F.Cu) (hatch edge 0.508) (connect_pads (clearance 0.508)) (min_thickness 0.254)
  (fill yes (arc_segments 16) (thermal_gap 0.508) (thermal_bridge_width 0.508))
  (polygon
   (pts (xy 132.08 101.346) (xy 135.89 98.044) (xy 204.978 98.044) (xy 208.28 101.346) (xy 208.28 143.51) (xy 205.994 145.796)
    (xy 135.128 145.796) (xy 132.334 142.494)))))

